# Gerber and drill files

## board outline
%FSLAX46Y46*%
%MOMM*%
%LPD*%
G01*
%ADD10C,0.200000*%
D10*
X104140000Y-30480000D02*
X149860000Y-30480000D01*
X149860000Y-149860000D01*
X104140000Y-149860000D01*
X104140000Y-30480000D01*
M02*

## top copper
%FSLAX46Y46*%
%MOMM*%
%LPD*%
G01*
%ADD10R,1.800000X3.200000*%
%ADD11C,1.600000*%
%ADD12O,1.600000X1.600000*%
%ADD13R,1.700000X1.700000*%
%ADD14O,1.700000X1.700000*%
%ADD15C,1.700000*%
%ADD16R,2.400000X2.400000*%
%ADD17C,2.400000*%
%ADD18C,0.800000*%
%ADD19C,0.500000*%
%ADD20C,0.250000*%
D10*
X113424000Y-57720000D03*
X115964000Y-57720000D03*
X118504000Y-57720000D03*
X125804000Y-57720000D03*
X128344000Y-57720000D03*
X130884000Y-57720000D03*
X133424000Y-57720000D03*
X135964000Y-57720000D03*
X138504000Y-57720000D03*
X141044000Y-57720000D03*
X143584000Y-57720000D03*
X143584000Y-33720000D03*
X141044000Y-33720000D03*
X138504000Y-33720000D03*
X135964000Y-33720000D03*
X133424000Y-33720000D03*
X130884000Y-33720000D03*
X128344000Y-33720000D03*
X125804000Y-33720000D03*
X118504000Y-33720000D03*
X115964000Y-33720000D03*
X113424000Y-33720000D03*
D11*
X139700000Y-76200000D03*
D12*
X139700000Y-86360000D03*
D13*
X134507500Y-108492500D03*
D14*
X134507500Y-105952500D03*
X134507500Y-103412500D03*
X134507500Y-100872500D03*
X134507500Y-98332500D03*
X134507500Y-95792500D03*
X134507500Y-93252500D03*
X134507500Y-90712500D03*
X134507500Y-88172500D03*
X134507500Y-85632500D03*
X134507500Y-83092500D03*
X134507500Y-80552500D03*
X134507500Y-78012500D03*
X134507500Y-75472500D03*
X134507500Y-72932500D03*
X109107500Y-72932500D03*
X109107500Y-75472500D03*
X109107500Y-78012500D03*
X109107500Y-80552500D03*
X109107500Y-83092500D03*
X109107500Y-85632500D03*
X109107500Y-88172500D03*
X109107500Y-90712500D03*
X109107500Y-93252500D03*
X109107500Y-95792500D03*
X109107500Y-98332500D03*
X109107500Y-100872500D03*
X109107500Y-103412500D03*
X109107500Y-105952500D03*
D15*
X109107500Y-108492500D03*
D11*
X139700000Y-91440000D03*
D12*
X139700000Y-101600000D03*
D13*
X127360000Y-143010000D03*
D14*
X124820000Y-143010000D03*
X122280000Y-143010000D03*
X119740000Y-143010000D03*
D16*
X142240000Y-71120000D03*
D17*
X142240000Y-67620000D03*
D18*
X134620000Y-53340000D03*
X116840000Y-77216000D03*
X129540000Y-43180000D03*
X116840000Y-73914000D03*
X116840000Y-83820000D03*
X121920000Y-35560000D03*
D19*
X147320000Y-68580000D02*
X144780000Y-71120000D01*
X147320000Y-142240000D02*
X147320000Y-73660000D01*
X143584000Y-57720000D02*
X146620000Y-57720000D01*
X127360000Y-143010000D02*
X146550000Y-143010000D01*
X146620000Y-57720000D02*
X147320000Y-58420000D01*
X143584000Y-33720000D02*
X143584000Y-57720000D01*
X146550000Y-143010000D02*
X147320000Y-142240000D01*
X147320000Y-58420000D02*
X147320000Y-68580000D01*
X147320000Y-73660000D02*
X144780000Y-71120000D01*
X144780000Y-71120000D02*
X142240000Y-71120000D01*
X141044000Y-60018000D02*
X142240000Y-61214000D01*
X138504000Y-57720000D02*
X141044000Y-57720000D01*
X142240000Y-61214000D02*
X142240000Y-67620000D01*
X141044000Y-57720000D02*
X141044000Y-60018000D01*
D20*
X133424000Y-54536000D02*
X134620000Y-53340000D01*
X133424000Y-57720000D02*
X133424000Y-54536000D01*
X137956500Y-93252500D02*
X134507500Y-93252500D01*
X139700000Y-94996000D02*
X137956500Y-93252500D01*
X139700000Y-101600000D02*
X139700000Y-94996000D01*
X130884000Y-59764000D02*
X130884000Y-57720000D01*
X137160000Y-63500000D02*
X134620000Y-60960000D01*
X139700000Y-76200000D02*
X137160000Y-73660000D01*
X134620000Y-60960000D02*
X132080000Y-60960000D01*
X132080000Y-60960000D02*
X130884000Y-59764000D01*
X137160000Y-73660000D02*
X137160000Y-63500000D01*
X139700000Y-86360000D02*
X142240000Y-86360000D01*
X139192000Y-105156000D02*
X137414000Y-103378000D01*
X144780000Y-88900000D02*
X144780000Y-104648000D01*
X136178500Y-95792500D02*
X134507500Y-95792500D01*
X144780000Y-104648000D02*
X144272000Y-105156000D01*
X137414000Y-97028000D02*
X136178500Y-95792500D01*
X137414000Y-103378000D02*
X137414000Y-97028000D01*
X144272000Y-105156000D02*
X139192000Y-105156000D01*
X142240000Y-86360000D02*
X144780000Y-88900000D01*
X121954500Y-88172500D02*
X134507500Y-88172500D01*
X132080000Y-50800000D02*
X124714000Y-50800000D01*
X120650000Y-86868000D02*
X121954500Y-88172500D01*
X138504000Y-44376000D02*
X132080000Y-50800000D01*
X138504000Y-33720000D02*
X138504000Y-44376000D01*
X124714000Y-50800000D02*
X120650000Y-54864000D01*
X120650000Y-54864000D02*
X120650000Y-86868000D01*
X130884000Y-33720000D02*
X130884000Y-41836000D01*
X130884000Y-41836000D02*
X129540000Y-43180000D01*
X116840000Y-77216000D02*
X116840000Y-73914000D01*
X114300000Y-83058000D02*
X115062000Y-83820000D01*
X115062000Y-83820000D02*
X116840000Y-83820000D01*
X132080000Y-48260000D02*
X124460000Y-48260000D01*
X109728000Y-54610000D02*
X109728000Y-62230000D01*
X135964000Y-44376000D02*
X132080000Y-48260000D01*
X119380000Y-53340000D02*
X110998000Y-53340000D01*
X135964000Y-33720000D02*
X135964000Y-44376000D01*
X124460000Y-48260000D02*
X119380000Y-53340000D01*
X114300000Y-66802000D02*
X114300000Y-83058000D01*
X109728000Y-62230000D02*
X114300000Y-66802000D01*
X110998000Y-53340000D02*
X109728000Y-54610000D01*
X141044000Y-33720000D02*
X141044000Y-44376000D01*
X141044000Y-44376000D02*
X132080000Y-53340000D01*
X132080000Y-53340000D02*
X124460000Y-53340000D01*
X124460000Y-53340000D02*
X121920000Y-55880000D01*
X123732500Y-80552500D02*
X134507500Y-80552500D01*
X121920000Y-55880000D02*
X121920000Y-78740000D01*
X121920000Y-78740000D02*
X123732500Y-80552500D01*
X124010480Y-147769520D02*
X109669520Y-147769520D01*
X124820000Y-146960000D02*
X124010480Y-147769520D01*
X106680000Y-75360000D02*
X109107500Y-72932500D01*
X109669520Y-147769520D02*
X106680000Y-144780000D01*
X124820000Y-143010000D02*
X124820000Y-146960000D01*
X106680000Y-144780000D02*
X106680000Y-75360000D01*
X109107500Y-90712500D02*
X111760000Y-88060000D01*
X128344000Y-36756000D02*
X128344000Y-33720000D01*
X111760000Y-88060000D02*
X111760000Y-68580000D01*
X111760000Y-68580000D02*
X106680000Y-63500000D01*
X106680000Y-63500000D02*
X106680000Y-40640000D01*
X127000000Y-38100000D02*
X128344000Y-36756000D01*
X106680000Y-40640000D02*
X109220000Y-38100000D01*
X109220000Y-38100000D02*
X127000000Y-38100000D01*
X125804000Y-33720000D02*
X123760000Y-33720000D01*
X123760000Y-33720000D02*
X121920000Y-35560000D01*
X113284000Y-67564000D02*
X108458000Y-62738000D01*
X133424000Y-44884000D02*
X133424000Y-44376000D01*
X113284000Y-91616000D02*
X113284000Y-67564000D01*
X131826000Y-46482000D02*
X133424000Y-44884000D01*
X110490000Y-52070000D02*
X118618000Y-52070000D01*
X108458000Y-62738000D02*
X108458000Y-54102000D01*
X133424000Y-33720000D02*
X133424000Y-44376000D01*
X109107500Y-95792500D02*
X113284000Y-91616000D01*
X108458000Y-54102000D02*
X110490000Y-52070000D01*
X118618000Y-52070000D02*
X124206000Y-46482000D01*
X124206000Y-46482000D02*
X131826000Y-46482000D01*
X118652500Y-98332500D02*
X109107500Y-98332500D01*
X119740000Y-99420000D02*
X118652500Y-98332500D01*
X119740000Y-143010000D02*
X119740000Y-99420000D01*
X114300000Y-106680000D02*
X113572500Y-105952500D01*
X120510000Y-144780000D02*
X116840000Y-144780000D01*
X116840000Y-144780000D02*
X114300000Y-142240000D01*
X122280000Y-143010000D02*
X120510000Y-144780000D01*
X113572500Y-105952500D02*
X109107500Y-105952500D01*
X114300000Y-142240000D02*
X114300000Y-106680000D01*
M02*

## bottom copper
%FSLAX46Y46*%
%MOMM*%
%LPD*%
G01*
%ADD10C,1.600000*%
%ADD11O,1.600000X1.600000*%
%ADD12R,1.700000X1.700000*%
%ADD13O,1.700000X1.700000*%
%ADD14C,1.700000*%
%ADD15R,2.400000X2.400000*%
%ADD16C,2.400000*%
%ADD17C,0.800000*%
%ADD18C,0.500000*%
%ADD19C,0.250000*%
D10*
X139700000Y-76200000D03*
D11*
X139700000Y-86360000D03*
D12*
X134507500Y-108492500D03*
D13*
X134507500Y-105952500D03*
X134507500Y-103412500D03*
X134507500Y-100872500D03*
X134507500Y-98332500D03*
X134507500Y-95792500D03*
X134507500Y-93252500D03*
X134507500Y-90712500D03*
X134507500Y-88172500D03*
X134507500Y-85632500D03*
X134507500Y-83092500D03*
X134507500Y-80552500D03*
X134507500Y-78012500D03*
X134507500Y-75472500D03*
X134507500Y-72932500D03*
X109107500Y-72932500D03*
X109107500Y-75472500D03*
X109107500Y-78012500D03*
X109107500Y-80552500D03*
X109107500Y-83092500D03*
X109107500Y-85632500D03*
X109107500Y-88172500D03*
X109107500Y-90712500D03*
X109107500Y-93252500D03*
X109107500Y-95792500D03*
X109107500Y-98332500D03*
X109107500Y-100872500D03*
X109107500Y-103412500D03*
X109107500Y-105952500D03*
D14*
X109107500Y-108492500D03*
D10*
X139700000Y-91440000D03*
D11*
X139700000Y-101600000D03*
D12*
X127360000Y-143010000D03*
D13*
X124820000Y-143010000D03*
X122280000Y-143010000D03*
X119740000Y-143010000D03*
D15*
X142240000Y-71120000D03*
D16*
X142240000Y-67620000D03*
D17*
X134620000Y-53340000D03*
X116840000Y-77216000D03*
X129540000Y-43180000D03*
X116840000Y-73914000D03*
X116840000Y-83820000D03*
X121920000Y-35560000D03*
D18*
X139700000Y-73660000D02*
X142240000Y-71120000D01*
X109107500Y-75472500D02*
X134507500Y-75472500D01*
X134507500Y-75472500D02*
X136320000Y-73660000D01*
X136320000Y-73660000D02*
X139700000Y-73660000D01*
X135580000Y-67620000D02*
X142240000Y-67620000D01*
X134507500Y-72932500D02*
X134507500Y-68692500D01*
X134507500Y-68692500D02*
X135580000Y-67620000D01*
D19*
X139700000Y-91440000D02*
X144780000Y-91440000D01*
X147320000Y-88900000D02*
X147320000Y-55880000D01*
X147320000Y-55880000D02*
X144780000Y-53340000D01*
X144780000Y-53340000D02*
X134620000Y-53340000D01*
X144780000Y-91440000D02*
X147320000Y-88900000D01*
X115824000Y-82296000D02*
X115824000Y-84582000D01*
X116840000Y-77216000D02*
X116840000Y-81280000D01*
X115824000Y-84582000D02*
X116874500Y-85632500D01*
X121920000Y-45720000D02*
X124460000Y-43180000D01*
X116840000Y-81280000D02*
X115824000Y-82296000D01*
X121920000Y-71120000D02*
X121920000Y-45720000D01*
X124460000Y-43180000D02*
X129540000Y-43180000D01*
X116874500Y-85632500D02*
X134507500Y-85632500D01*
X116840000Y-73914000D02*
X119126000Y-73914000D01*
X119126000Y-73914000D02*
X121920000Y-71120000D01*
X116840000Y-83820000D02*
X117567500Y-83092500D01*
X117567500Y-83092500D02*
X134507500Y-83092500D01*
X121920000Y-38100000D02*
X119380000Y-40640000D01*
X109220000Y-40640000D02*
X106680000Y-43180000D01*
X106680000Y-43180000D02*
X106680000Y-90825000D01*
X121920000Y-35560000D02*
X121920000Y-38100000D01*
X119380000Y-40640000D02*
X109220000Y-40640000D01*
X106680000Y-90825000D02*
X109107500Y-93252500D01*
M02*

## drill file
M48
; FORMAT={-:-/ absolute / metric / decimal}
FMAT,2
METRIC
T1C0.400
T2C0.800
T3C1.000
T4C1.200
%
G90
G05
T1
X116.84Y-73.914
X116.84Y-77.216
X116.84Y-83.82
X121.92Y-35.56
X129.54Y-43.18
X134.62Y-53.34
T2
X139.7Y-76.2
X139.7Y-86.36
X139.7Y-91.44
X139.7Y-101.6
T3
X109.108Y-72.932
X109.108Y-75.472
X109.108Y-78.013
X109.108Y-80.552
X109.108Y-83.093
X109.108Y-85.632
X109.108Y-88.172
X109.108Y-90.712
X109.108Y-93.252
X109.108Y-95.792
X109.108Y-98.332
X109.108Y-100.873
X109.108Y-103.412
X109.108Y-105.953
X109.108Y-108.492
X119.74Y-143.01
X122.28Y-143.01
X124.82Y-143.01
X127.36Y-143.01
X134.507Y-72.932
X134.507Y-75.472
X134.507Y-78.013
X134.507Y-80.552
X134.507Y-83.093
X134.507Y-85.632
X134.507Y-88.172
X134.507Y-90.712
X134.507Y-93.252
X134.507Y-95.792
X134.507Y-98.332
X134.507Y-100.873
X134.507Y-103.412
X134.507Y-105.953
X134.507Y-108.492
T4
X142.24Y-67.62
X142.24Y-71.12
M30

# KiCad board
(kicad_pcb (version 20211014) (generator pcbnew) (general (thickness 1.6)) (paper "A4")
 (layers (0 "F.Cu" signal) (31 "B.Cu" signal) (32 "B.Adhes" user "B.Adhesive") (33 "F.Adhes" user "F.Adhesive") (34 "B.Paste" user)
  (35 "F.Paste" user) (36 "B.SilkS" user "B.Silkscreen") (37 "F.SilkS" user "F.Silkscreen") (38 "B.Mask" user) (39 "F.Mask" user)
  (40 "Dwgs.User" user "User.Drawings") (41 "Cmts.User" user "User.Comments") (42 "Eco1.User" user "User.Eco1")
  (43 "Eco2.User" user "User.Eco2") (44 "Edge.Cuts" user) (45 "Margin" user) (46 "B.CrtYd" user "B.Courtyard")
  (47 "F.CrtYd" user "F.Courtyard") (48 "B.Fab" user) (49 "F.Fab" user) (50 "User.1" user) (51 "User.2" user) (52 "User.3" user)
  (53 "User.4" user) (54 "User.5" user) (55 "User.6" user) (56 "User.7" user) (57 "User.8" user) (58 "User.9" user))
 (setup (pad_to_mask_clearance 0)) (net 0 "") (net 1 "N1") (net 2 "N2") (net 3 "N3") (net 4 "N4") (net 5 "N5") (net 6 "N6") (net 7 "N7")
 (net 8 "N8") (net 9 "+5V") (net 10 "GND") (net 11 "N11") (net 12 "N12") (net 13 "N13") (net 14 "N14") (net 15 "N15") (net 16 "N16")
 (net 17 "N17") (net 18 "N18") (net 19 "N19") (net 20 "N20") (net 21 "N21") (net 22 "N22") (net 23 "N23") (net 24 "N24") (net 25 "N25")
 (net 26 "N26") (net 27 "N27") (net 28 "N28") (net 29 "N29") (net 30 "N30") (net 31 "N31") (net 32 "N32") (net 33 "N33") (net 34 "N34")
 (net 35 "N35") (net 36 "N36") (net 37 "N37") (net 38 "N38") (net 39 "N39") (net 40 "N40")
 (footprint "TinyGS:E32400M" (layer "F.Cu") (at 146.155 33.72 -90)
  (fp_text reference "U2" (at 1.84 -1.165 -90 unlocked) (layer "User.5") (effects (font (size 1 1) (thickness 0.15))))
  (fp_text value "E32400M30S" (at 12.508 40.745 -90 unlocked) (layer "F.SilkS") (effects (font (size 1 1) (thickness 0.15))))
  (pad "1" smd rect (at 24 32.731 270) (size 3.2 1.8) (layers "F.Cu" "F.Paste" "F.Mask") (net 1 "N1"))
  (pad "2" smd rect (at 24 30.191 270) (size 3.2 1.8) (layers "F.Cu" "F.Paste" "F.Mask") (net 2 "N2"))
  (pad "3" smd rect (at 24 27.651 270) (size 3.2 1.8) (layers "F.Cu" "F.Paste" "F.Mask") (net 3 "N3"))
  (pad "4" smd rect (at 24 20.351 270) (size 3.2 1.8) (layers "F.Cu" "F.Paste" "F.Mask") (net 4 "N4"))
  (pad "5" smd rect (at 24 17.811 270) (size 3.2 1.8) (layers "F.Cu" "F.Paste" "F.Mask") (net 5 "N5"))
  (pad "6" smd rect (at 24 15.271 270) (size 3.2 1.8) (layers "F.Cu" "F.Paste" "F.Mask") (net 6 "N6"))
  (pad "7" smd rect (at 24 12.731 270) (size 3.2 1.8) (layers "F.Cu" "F.Paste" "F.Mask") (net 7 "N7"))
  (pad "8" smd rect (at 24 10.191 270) (size 3.2 1.8) (layers "F.Cu" "F.Paste" "F.Mask") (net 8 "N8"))
  (pad "9" smd rect (at 24 7.651 270) (size 3.2 1.8) (layers "F.Cu" "F.Paste" "F.Mask") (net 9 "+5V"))
  (pad "10" smd rect (at 24 5.111 270) (size 3.2 1.8) (layers "F.Cu" "F.Paste" "F.Mask") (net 9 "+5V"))
  (pad "11" smd rect (at 24 2.571 270) (size 3.2 1.8) (layers "F.Cu" "F.Paste" "F.Mask") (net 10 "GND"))
  (pad "18" smd rect (at 0 2.571 270) (size 3.2 1.8) (layers "F.Cu" "F.Paste" "F.Mask") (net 10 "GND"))
  (pad "19" smd rect (at 0 5.111 270) (size 3.2 1.8) (layers "F.Cu" "F.Paste" "F.Mask") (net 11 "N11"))
  (pad "20" smd rect (at 0 7.651 270) (size 3.2 1.8) (layers "F.Cu" "F.Paste" "F.Mask") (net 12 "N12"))
  (pad "21" smd rect (at 0 10.191 270) (size 3.2 1.8) (layers "F.Cu" "F.Paste" "F.Mask") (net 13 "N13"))
  (pad "22" smd rect (at 0 12.731 270) (size 3.2 1.8) (layers "F.Cu" "F.Paste" "F.Mask") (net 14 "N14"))
  (pad "23" smd rect (at 0 15.271 270) (size 3.2 1.8) (layers "F.Cu" "F.Paste" "F.Mask") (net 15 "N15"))
  (pad "24" smd rect (at 0 17.811 270) (size 3.2 1.8) (layers "F.Cu" "F.Paste" "F.Mask") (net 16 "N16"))
  (pad "25" smd rect (at 0 20.351 270) (size 3.2 1.8) (layers "F.Cu" "F.Paste" "F.Mask") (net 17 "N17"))
  (pad "26" smd rect (at 0 27.651 270) (size 3.2 1.8) (layers "F.Cu" "F.Paste" "F.Mask") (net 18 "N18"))
  (pad "27" smd rect (at 0 30.191 270) (size 3.2 1.8) (layers "F.Cu" "F.Paste" "F.Mask") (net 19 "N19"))
  (pad "28" smd rect (at 0 32.731 270) (size 3.2 1.8) (layers "F.Cu" "F.Paste" "F.Mask") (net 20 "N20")))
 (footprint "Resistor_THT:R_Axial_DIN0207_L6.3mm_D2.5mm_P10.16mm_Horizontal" (layer "F.Cu") (at 139.7 76.2 -90)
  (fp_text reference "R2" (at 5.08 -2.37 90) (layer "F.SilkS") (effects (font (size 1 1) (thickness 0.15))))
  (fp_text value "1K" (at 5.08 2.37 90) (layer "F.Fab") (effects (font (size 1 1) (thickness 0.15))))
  (pad "1" thru_hole circle (at 0 0 270) (size 1.6 1.6) (drill 0.8) (layers *.Cu *.Mask) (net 6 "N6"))
  (pad "2" thru_hole oval (at 10.16 0 270) (size 1.6 1.6) (drill 0.8) (layers *.Cu *.Mask) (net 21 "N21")))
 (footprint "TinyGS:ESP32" (layer "F.Cu") (at 136.0575 114.5125 180)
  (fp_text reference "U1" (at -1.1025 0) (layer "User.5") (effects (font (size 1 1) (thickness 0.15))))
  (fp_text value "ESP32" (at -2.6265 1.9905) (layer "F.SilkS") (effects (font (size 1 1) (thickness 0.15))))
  (pad "1" thru_hole rect (at 1.55 6.02 180) (size 1.7 1.7) (drill 1) (layers *.Cu *.Mask) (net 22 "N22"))
  (pad "2" thru_hole oval (at 1.55 8.56 180) (size 1.7 1.7) (drill 1) (layers *.Cu *.Mask) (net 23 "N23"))
  (pad "3" thru_hole oval (at 1.55 11.1 180) (size 1.7 1.7) (drill 1) (layers *.Cu *.Mask) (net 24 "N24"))
  (pad "4" thru_hole oval (at 1.55 13.64 180) (size 1.7 1.7) (drill 1) (layers *.Cu *.Mask) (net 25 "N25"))
  (pad "5" thru_hole oval (at 1.55 16.18 180) (size 1.7 1.7) (drill 1) (layers *.Cu *.Mask) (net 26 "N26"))
  (pad "6" thru_hole oval (at 1.55 18.72 180) (size 1.7 1.7) (drill 1) (layers *.Cu *.Mask) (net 21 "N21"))
  (pad "7" thru_hole oval (at 1.55 21.26 180) (size 1.7 1.7) (drill 1) (layers *.Cu *.Mask) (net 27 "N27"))
  (pad "8" thru_hole oval (at 1.55 23.8 180) (size 1.7 1.7) (drill 1) (layers *.Cu *.Mask) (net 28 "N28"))
  (pad "9" thru_hole oval (at 1.55 26.34 180) (size 1.7 1.7) (drill 1) (layers *.Cu *.Mask) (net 12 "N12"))
  (pad "10" thru_hole oval (at 1.55 28.88 180) (size 1.7 1.7) (drill 1) (layers *.Cu *.Mask) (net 15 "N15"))
  (pad "11" thru_hole oval (at 1.55 31.42 180) (size 1.7 1.7) (drill 1) (layers *.Cu *.Mask) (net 13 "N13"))
  (pad "12" thru_hole oval (at 1.55 33.96 180) (size 1.7 1.7) (drill 1) (layers *.Cu *.Mask) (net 11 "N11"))
  (pad "13" thru_hole oval (at 1.55 36.5 180) (size 1.7 1.7) (drill 1) (layers *.Cu *.Mask) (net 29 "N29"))
  (pad "14" thru_hole oval (at 1.55 39.04 180) (size 1.7 1.7) (drill 1) (layers *.Cu *.Mask) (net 10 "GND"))
  (pad "15" thru_hole oval (at 1.55 41.58 180) (size 1.7 1.7) (drill 1) (layers *.Cu *.Mask) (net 9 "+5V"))
  (pad "16" thru_hole oval (at 26.95 41.58 180) (size 1.7 1.7) (drill 1) (layers *.Cu *.Mask) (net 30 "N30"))
  (pad "17" thru_hole oval (at 26.95 39.04 180) (size 1.7 1.7) (drill 1) (layers *.Cu *.Mask) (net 10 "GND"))
  (pad "18" thru_hole oval (at 26.95 36.5 180) (size 1.7 1.7) (drill 1) (layers *.Cu *.Mask) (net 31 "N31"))
  (pad "19" thru_hole oval (at 26.95 33.96 180) (size 1.7 1.7) (drill 1) (layers *.Cu *.Mask) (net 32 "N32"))
  (pad "20" thru_hole oval (at 26.95 31.42 180) (size 1.7 1.7) (drill 1) (layers *.Cu *.Mask) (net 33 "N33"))
  (pad "21" thru_hole oval (at 26.95 28.88 180) (size 1.7 1.7) (drill 1) (layers *.Cu *.Mask) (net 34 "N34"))
  (pad "22" thru_hole oval (at 26.95 26.34 180) (size 1.7 1.7) (drill 1) (layers *.Cu *.Mask) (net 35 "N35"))
  (pad "23" thru_hole oval (at 26.95 23.8 180) (size 1.7 1.7) (drill 1) (layers *.Cu *.Mask) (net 16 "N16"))
  (pad "24" thru_hole oval (at 26.95 21.26 180) (size 1.7 1.7) (drill 1) (layers *.Cu *.Mask) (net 17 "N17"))
  (pad "25" thru_hole oval (at 26.95 18.72 180) (size 1.7 1.7) (drill 1) (layers *.Cu *.Mask) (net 14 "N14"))
  (pad "26" thru_hole oval (at 26.95 16.18 180) (size 1.7 1.7) (drill 1) (layers *.Cu *.Mask) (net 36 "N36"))
  (pad "27" thru_hole oval (at 26.95 13.64 180) (size 1.7 1.7) (drill 1) (layers *.Cu *.Mask) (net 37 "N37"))
  (pad "28" thru_hole oval (at 26.95 11.1 180) (size 1.7 1.7) (drill 1) (layers *.Cu *.Mask) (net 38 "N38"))
  (pad "29" thru_hole oval (at 26.95 8.56 180) (size 1.7 1.7) (drill 1) (layers *.Cu *.Mask) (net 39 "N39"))
  (pad "30" thru_hole circle (at 26.95 6.02 180) (size 1.7 1.7) (drill 1) (layers *.Cu *.Mask) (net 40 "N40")))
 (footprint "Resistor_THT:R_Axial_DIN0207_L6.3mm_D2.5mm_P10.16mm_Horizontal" (layer "F.Cu") (at 139.7 91.44 -90)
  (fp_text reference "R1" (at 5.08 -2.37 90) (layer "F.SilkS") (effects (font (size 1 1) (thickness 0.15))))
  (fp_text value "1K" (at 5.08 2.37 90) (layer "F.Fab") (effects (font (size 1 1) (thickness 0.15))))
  (pad "1" thru_hole circle (at 0 0 270) (size 1.6 1.6) (drill 0.8) (layers *.Cu *.Mask) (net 7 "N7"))
  (pad "2" thru_hole oval (at 10.16 0 270) (size 1.6 1.6) (drill 0.8) (layers *.Cu *.Mask) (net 27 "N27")))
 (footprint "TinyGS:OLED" (layer "F.Cu") (at 137.16 144.78 180)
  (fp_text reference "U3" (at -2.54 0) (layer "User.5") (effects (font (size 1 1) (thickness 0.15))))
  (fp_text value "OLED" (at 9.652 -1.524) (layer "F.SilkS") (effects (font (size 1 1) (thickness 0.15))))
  (pad "1" thru_hole rect (at 9.8 1.77 270) (size 1.7 1.7) (drill 1) (layers *.Cu *.Mask) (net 10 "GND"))
  (pad "2" thru_hole oval (at 12.34 1.77 270) (size 1.7 1.7) (drill 1) (layers *.Cu *.Mask) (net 30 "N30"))
  (pad "3" thru_hole oval (at 14.88 1.77 270) (size 1.7 1.7) (drill 1) (layers *.Cu *.Mask) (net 39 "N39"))
  (pad "4" thru_hole oval (at 17.42 1.77 270) (size 1.7 1.7) (drill 1) (layers *.Cu *.Mask) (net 36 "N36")))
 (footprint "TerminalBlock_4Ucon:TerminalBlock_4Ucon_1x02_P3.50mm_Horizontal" (layer "F.Cu") (at 142.24 71.12 90)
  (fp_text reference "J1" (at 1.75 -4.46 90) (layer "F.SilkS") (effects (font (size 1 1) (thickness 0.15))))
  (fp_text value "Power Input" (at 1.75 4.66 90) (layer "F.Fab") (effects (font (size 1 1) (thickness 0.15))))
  (pad "1" thru_hole rect (at 0 0 90) (size 2.4 2.4) (drill 1.2) (layers *.Cu *.Mask) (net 10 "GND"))
  (pad "2" thru_hole circle (at 3.5 0 90) (size 2.4 2.4) (drill 1.2) (layers *.Cu *.Mask) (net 9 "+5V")))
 (gr_rect (start 149.86 149.86) (end 104.14 30.48) (layer "Edge.Cuts") (width 0.2) (fill none))
 (segment (start 147.32 68.58) (end 144.78 71.12) (width 0.5) (layer "F.Cu") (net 10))
 (segment (start 147.32 142.24) (end 147.32 73.66) (width 0.5) (layer "F.Cu") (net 10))
 (segment (start 143.584 57.72) (end 146.62 57.72) (width 0.5) (layer "F.Cu") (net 10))
 (segment (start 127.36 143.01) (end 146.55 143.01) (width 0.5) (layer "F.Cu") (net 10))
 (segment (start 146.62 57.72) (end 147.32 58.42) (width 0.5) (layer "F.Cu") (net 10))
 (segment (start 143.584 33.72) (end 143.584 57.72) (width 0.5) (layer "F.Cu") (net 10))
 (segment (start 146.55 143.01) (end 147.32 142.24) (width 0.5) (layer "F.Cu") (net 10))
 (segment (start 147.32 58.42) (end 147.32 68.58) (width 0.5) (layer "F.Cu") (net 10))
 (segment (start 147.32 73.66) (end 144.78 71.12) (width 0.5) (layer "F.Cu") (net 10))
 (segment (start 144.78 71.12) (end 142.24 71.12) (width 0.5) (layer "F.Cu") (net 10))
 (segment (start 139.7 73.66) (end 142.24 71.12) (width 0.5) (layer "B.Cu") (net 10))
 (segment (start 109.1075 75.4725) (end 134.5075 75.4725) (width 0.5) (layer "B.Cu") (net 10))
 (segment (start 134.5075 75.4725) (end 136.32 73.66) (width 0.5) (layer "B.Cu") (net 10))
 (segment (start 136.32 73.66) (end 139.7 73.66) (width 0.5) (layer "B.Cu") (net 10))
 (segment (start 141.044 60.018) (end 142.24 61.214) (width 0.5) (layer "F.Cu") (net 9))
 (segment (start 138.504 57.72) (end 141.044 57.72) (width 0.5) (layer "F.Cu") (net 9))
 (segment (start 142.24 61.214) (end 142.24 67.62) (width 0.5) (layer "F.Cu") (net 9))
 (segment (start 141.044 57.72) (end 141.044 60.018) (width 0.5) (layer "F.Cu") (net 9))
 (segment (start 135.58 67.62) (end 142.24 67.62) (width 0.5) (layer "B.Cu") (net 9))
 (segment (start 134.5075 72.9325) (end 134.5075 68.6925) (width 0.5) (layer "B.Cu") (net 9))
 (segment (start 134.5075 68.6925) (end 135.58 67.62) (width 0.5) (layer "B.Cu") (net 9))
 (segment (start 133.424 54.536) (end 134.62 53.34) (width 0.25) (layer "F.Cu") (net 7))
 (segment (start 133.424 57.72) (end 133.424 54.536) (width 0.25) (layer "F.Cu") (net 7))
 (via (at 134.62 53.34) (size 0.8) (drill 0.4) (layers "F.Cu" "B.Cu") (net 7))
 (segment (start 139.7 91.44) (end 144.78 91.44) (width 0.25) (layer "B.Cu") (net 7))
 (segment (start 147.32 88.9) (end 147.32 55.88) (width 0.25) (layer "B.Cu") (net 7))
 (segment (start 147.32 55.88) (end 144.78 53.34) (width 0.25) (layer "B.Cu") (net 7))
 (segment (start 144.78 53.34) (end 134.62 53.34) (width 0.25) (layer "B.Cu") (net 7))
 (segment (start 144.78 91.44) (end 147.32 88.9) (width 0.25) (layer "B.Cu") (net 7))
 (segment (start 137.9565 93.2525) (end 134.5075 93.2525) (width 0.25) (layer "F.Cu") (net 27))
 (segment (start 139.7 94.996) (end 137.9565 93.2525) (width 0.25) (layer "F.Cu") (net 27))
 (segment (start 139.7 101.6) (end 139.7 94.996) (width 0.25) (layer "F.Cu") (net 27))
 (segment (start 130.884 59.764) (end 130.884 57.72) (width 0.25) (layer "F.Cu") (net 6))
 (segment (start 137.16 63.5) (end 134.62 60.96) (width 0.25) (layer "F.Cu") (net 6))
 (segment (start 139.7 76.2) (end 137.16 73.66) (width 0.25) (layer "F.Cu") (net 6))
 (segment (start 134.62 60.96) (end 132.08 60.96) (width 0.25) (layer "F.Cu") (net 6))
 (segment (start 132.08 60.96) (end 130.884 59.764) (width 0.25) (layer "F.Cu") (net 6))
 (segment (start 137.16 73.66) (end 137.16 63.5) (width 0.25) (layer "F.Cu") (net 6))
 (segment (start 139.7 86.36) (end 142.24 86.36) (width 0.25) (layer "F.Cu") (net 21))
 (segment (start 139.192 105.156) (end 137.414 103.378) (width 0.25) (layer "F.Cu") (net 21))
 (segment (start 144.78 88.9) (end 144.78 104.648) (width 0.25) (layer "F.Cu") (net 21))
 (segment (start 136.1785 95.7925) (end 134.5075 95.7925) (width 0.25) (layer "F.Cu") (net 21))
 (segment (start 144.78 104.648) (end 144.272 105.156) (width 0.25) (layer "F.Cu") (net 21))
 (segment (start 137.414 97.028) (end 136.1785 95.7925) (width 0.25) (layer "F.Cu") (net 21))
 (segment (start 137.414 103.378) (end 137.414 97.028) (width 0.25) (layer "F.Cu") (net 21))
 (segment (start 144.272 105.156) (end 139.192 105.156) (width 0.25) (layer "F.Cu") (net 21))
 (segment (start 142.24 86.36) (end 144.78 88.9) (width 0.25) (layer "F.Cu") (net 21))
 (segment (start 121.9545 88.1725) (end 134.5075 88.1725) (width 0.25) (layer "F.Cu") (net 12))
 (segment (start 132.08 50.8) (end 124.714 50.8) (width 0.25) (layer "F.Cu") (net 12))
 (segment (start 120.65 86.868) (end 121.9545 88.1725) (width 0.25) (layer "F.Cu") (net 12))
 (segment (start 138.504 44.376) (end 132.08 50.8) (width 0.25) (layer "F.Cu") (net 12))
 (segment (start 138.504 33.72) (end 138.504 44.376) (width 0.25) (layer "F.Cu") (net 12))
 (segment (start 124.714 50.8) (end 120.65 54.864) (width 0.25) (layer "F.Cu") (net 12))
 (segment (start 120.65 54.864) (end 120.65 86.868) (width 0.25) (layer "F.Cu") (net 12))
 (segment (start 130.884 33.72) (end 130.884 41.836) (width 0.25) (layer "F.Cu") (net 15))
 (segment (start 130.884 41.836) (end 129.54 43.18) (width 0.25) (layer "F.Cu") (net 15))
 (segment (start 116.84 77.216) (end 116.84 73.914) (width 0.25) (layer "F.Cu") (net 15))
 (via (at 116.84 77.216) (size 0.8) (drill 0.4) (layers "F.Cu" "B.Cu") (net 15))
 (via (at 129.54 43.18) (size 0.8) (drill 0.4) (layers "F.Cu" "B.Cu") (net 15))
 (via (at 116.84 73.914) (size 0.8) (drill 0.4) (layers "F.Cu" "B.Cu") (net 15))
 (segment (start 115.824 82.296) (end 115.824 84.582) (width 0.25) (layer "B.Cu") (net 15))
 (segment (start 116.84 77.216) (end 116.84 81.28) (width 0.25) (layer "B.Cu") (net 15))
 (segment (start 115.824 84.582) (end 116.8745 85.6325) (width 0.25) (layer "B.Cu") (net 15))
 (segment (start 121.92 45.72) (end 124.46 43.18) (width 0.25) (layer "B.Cu") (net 15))
 (segment (start 116.84 81.28) (end 115.824 82.296) (width 0.25) (layer "B.Cu") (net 15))
 (segment (start 121.92 71.12) (end 121.92 45.72) (width 0.25) (layer "B.Cu") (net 15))
 (segment (start 124.46 43.18) (end 129.54 43.18) (width 0.25) (layer "B.Cu") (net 15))
 (segment (start 116.8745 85.6325) (end 134.5075 85.6325) (width 0.25) (layer "B.Cu") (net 15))
 (segment (start 116.84 73.914) (end 119.126 73.914) (width 0.25) (layer "B.Cu") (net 15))
 (segment (start 119.126 73.914) (end 121.92 71.12) (width 0.25) (layer "B.Cu") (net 15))
 (segment (start 114.3 83.058) (end 115.062 83.82) (width 0.25) (layer "F.Cu") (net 13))
 (segment (start 115.062 83.82) (end 116.84 83.82) (width 0.25) (layer "F.Cu") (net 13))
 (segment (start 132.08 48.26) (end 124.46 48.26) (width 0.25) (layer "F.Cu") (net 13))
 (segment (start 109.728 54.61) (end 109.728 62.23) (width 0.25) (layer "F.Cu") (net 13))
 (segment (start 135.964 44.376) (end 132.08 48.26) (width 0.25) (layer "F.Cu") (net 13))
 (segment (start 119.38 53.34) (end 110.998 53.34) (width 0.25) (layer "F.Cu") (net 13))
 (segment (start 135.964 33.72) (end 135.964 44.376) (width 0.25) (layer "F.Cu") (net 13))
 (segment (start 124.46 48.26) (end 119.38 53.34) (width 0.25) (layer "F.Cu") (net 13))
 (segment (start 114.3 66.802) (end 114.3 83.058) (width 0.25) (layer "F.Cu") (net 13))
 (segment (start 109.728 62.23) (end 114.3 66.802) (width 0.25) (layer "F.Cu") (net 13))
 (segment (start 110.998 53.34) (end 109.728 54.61) (width 0.25) (layer "F.Cu") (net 13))
 (via (at 116.84 83.82) (size 0.8) (drill 0.4) (layers "F.Cu" "B.Cu") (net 13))
 (segment (start 116.84 83.82) (end 117.5675 83.0925) (width 0.25) (layer "B.Cu") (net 13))
 (segment (start 117.5675 83.0925) (end 134.5075 83.0925) (width 0.25) (layer "B.Cu") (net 13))
 (segment (start 141.044 33.72) (end 141.044 44.376) (width 0.25) (layer "F.Cu") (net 11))
 (segment (start 141.044 44.376) (end 132.08 53.34) (width 0.25) (layer "F.Cu") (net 11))
 (segment (start 132.08 53.34) (end 124.46 53.34) (width 0.25) (layer "F.Cu") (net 11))
 (segment (start 124.46 53.34) (end 121.92 55.88) (width 0.25) (layer "F.Cu") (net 11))
 (segment (start 123.7325 80.5525) (end 134.5075 80.5525) (width 0.25) (layer "F.Cu") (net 11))
 (segment (start 121.92 55.88) (end 121.92 78.74) (width 0.25) (layer "F.Cu") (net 11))
 (segment (start 121.92 78.74) (end 123.7325 80.5525) (width 0.25) (layer "F.Cu") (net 11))
 (segment (start 124.01048 147.76952) (end 109.66952 147.76952) (width 0.25) (layer "F.Cu") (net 30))
 (segment (start 124.82 146.96) (end 124.01048 147.76952) (width 0.25) (layer "F.Cu") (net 30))
 (segment (start 106.68 75.36) (end 109.1075 72.9325) (width 0.25) (layer "F.Cu") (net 30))
 (segment (start 109.66952 147.76952) (end 106.68 144.78) (width 0.25) (layer "F.Cu") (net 30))
 (segment (start 124.82 143.01) (end 124.82 146.96) (width 0.25) (layer "F.Cu") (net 30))
 (segment (start 106.68 144.78) (end 106.68 75.36) (width 0.25) (layer "F.Cu") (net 30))
 (segment (start 109.1075 90.7125) (end 111.76 88.06) (width 0.25) (layer "F.Cu") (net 16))
 (segment (start 128.344 36.756) (end 128.344 33.72) (width 0.25) (layer "F.Cu") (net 16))
 (segment (start 111.76 88.06) (end 111.76 68.58) (width 0.25) (layer "F.Cu") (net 16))
 (segment (start 111.76 68.58) (end 106.68 63.5) (width 0.25) (layer "F.Cu") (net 16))
 (segment (start 106.68 63.5) (end 106.68 40.64) (width 0.25) (layer "F.Cu") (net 16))
 (segment (start 127 38.1) (end 128.344 36.756) (width 0.25) (layer "F.Cu") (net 16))
 (segment (start 106.68 40.64) (end 109.22 38.1) (width 0.25) (layer "F.Cu") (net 16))
 (segment (start 109.22 38.1) (end 127 38.1) (width 0.25) (layer "F.Cu") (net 16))
 (segment (start 125.804 33.72) (end 123.76 33.72) (width 0.25) (layer "F.Cu") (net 17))
 (segment (start 123.76 33.72) (end 121.92 35.56) (width 0.25) (layer "F.Cu") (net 17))
 (via (at 121.92 35.56) (size 0.8) (drill 0.4) (layers "F.Cu" "B.Cu") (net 17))
 (segment (start 121.92 38.1) (end 119.38 40.64) (width 0.25) (layer "B.Cu") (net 17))
 (segment (start 109.22 40.64) (end 106.68 43.18) (width 0.25) (layer "B.Cu") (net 17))
 (segment (start 106.68 43.18) (end 106.68 90.825) (width 0.25) (layer "B.Cu") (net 17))
 (segment (start 121.92 35.56) (end 121.92 38.1) (width 0.25) (layer "B.Cu") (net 17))
 (segment (start 119.38 40.64) (end 109.22 40.64) (width 0.25) (layer "B.Cu") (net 17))
 (segment (start 106.68 90.825) (end 109.1075 93.2525) (width 0.25) (layer "B.Cu") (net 17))
 (segment (start 113.284 67.564) (end 108.458 62.738) (width 0.25) (layer "F.Cu") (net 14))
 (segment (start 133.424 44.884) (end 133.424 44.376) (width 0.25) (layer "F.Cu") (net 14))
 (segment (start 113.284 91.616) (end 113.284 67.564) (width 0.25) (layer "F.Cu") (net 14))
 (segment (start 131.826 46.482) (end 133.424 44.884) (width 0.25) (layer "F.Cu") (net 14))
 (segment (start 110.49 52.07) (end 118.618 52.07) (width 0.25) (layer "F.Cu") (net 14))
 (segment (start 108.458 62.738) (end 108.458 54.102) (width 0.25) (layer "F.Cu") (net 14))
 (segment (start 133.424 33.72) (end 133.424 44.376) (width 0.25) (layer "F.Cu") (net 14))
 (segment (start 109.1075 95.7925) (end 113.284 91.616) (width 0.25) (layer "F.Cu") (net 14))
 (segment (start 108.458 54.102) (end 110.49 52.07) (width 0.25) (layer "F.Cu") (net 14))
 (segment (start 118.618 52.07) (end 124.206 46.482) (width 0.25) (layer "F.Cu") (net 14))
 (segment (start 124.206 46.482) (end 131.826 46.482) (width 0.25) (layer "F.Cu") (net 14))
 (segment (start 118.6525 98.3325) (end 109.1075 98.3325) (width 0.25) (layer "F.Cu") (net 36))
 (segment (start 119.74 99.42) (end 118.6525 98.3325) (width 0.25) (layer "F.Cu") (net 36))
 (segment (start 119.74 143.01) (end 119.74 99.42) (width 0.25) (layer "F.Cu") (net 36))
 (segment (start 114.3 106.68) (end 113.5725 105.9525) (width 0.25) (layer "F.Cu") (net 39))
 (segment (start 120.51 144.78) (end 116.84 144.78) (width 0.25) (layer "F.Cu") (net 39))
 (segment (start 116.84 144.78) (end 114.3 142.24) (width 0.25) (layer "F.Cu") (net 39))
 (segment (start 122.28 143.01) (end 120.51 144.78) (width 0.25) (layer "F.Cu") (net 39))
 (segment (start 113.5725 105.9525) (end 109.1075 105.9525) (width 0.25) (layer "F.Cu") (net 39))
 (segment (start 114.3 142.24) (end 114.3 106.68) (width 0.25) (layer "F.Cu") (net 39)))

